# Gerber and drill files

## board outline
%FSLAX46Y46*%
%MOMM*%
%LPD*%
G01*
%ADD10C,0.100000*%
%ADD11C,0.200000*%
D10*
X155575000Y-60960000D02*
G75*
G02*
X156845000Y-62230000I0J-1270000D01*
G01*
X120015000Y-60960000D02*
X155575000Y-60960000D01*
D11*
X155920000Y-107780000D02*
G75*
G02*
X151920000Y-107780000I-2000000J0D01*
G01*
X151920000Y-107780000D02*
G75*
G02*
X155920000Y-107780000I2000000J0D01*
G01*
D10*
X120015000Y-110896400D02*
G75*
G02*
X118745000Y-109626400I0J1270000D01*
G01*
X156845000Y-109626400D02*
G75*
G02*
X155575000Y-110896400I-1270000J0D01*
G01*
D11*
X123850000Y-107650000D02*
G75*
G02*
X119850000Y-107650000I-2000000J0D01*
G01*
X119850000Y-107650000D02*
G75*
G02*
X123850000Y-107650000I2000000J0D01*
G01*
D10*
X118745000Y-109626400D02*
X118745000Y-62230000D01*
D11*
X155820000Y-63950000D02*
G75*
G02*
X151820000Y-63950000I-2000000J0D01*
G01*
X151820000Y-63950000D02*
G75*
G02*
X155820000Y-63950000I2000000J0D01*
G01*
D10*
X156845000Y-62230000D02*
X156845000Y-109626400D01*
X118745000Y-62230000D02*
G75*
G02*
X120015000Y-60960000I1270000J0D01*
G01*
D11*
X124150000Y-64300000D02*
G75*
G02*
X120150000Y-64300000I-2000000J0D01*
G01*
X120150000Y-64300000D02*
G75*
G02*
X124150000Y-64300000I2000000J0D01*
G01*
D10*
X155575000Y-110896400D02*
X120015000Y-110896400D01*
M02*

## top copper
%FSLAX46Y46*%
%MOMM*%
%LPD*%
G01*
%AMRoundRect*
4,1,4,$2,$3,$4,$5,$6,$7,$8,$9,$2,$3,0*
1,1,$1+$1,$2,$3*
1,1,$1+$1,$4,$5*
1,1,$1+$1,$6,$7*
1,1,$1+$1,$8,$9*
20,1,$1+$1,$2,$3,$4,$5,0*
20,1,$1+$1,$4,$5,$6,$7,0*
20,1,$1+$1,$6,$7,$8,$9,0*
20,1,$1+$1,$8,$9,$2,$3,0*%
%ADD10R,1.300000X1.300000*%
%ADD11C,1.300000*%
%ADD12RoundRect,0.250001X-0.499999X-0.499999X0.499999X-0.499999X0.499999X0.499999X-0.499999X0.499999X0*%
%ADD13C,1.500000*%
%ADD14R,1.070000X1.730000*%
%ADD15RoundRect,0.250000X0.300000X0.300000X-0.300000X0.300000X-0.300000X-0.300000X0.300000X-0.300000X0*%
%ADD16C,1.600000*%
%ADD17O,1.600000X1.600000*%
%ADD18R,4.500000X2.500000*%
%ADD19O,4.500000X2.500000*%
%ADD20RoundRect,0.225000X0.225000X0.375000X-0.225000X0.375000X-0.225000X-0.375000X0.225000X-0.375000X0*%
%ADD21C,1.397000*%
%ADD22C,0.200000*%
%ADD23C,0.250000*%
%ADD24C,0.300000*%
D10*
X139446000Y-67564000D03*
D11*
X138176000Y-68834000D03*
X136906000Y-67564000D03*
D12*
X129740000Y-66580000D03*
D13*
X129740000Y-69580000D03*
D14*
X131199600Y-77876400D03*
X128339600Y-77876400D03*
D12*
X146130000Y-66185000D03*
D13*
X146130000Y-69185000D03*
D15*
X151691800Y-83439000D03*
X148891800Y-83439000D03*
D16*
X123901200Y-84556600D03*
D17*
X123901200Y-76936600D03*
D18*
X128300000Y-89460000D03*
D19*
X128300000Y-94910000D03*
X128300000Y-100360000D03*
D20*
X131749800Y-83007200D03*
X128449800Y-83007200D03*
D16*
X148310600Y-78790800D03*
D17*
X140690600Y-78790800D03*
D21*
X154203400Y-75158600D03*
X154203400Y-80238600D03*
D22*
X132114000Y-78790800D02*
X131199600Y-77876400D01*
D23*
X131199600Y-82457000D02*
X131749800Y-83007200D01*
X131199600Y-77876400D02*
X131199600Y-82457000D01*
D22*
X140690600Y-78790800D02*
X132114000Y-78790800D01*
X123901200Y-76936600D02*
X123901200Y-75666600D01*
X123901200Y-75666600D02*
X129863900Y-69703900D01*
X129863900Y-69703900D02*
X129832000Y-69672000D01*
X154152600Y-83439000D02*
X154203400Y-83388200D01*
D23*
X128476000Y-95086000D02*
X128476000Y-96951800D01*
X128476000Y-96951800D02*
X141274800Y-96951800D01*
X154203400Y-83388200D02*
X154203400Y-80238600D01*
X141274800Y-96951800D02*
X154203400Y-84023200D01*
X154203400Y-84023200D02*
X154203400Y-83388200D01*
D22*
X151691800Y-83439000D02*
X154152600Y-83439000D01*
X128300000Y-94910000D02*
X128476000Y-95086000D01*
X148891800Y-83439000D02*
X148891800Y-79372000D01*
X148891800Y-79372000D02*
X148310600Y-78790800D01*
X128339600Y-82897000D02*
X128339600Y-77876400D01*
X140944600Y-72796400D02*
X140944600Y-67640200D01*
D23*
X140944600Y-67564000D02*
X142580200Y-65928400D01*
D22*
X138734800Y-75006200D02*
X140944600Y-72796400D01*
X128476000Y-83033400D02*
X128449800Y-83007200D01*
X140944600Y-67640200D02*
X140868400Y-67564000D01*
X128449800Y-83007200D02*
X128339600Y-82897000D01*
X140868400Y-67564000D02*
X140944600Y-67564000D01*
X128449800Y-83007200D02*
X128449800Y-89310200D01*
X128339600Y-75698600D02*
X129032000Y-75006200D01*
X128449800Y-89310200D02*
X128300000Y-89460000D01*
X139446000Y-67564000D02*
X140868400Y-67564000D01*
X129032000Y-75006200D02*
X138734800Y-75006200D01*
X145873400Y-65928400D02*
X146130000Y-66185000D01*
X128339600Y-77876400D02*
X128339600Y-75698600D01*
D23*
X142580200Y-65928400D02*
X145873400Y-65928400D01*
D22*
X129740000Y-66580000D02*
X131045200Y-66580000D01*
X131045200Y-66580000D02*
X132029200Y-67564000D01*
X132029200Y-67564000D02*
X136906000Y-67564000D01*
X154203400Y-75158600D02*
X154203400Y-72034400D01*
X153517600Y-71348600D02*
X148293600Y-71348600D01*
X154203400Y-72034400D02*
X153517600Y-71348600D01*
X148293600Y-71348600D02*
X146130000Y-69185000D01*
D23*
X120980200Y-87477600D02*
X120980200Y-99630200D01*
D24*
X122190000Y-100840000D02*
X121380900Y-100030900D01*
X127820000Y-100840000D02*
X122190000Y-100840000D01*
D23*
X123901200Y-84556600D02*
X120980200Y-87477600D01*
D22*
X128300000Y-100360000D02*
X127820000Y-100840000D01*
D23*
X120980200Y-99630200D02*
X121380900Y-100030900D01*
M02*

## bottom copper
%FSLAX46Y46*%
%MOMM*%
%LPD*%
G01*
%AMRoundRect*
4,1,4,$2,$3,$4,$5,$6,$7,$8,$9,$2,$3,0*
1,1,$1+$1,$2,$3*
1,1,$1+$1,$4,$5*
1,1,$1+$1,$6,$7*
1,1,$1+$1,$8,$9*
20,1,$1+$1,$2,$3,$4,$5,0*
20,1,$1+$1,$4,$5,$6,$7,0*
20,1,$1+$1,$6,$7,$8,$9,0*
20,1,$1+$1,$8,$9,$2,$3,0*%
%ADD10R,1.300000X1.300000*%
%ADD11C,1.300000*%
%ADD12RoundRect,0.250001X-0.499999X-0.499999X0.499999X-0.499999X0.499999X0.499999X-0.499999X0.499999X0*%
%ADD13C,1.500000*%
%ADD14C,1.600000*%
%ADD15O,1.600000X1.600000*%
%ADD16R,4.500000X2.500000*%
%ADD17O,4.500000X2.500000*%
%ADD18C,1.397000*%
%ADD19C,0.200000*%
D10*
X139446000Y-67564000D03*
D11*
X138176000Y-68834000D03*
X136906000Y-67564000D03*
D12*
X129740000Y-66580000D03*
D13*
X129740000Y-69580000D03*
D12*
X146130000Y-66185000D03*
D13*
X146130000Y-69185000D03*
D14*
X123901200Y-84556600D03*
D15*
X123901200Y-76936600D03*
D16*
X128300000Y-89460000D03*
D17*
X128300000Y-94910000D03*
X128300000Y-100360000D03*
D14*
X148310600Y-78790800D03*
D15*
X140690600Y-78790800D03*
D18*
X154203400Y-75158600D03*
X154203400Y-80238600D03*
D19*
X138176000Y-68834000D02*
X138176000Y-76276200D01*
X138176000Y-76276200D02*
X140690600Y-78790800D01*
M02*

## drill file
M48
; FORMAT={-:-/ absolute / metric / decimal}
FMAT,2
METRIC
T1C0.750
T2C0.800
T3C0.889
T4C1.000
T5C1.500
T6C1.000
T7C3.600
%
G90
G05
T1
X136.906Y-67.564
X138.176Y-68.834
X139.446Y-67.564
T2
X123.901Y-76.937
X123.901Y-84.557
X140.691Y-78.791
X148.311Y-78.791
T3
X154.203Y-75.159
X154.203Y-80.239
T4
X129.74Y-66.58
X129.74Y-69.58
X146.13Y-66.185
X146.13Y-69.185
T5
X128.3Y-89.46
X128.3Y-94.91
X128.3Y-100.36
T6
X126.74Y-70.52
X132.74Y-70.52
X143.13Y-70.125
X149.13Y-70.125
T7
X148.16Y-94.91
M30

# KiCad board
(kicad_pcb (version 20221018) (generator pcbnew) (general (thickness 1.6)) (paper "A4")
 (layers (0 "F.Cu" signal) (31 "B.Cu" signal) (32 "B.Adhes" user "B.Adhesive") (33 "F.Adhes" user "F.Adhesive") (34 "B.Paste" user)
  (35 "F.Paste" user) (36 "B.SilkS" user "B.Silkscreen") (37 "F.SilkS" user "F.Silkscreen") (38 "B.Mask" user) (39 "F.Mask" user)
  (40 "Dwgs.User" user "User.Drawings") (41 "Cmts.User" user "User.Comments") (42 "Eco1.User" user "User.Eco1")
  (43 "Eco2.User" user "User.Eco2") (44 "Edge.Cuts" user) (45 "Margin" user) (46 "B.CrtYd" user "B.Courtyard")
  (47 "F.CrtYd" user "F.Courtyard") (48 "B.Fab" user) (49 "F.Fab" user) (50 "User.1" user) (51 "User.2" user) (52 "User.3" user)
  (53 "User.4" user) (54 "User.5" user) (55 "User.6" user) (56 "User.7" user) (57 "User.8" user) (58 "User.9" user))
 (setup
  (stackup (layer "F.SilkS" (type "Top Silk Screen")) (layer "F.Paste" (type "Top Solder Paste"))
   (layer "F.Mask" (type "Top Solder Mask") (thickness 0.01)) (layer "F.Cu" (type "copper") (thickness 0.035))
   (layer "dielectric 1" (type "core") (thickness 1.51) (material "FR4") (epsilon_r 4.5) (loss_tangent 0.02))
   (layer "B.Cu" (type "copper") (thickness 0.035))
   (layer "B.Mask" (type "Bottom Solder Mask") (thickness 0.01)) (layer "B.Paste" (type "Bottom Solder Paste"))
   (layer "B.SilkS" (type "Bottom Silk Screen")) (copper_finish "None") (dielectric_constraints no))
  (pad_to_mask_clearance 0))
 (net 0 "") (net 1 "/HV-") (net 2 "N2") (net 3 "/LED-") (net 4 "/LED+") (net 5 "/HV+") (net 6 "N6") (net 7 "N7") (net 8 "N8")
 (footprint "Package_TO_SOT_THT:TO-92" (layer "F.Cu") (at 139.446 67.564 180)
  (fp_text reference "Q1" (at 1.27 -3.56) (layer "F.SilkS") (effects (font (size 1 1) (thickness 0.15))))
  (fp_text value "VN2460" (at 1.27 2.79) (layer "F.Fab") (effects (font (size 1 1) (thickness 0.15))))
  (pad "1" thru_hole rect (at 0 0 180) (size 1.3 1.3) (drill 0.75) (layers "*.Cu" "*.Mask") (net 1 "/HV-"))
  (pad "2" thru_hole circle (at 1.27 -1.27 180) (size 1.3 1.3) (drill 0.75) (layers "*.Cu" "*.Mask") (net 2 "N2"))
  (pad "3" thru_hole circle (at 2.54 0 180) (size 1.3 1.3) (drill 0.75) (layers "*.Cu" "*.Mask") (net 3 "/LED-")))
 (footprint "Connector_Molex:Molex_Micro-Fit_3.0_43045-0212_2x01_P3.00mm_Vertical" (layer "F.Cu") (at 129.74 66.58)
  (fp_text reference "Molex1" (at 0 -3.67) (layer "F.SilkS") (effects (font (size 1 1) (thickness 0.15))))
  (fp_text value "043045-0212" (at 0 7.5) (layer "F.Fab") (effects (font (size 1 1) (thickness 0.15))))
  (pad "" np_thru_hole circle (at -3 3.94) (size 1 1) (drill 1) (layers "*.Cu" "*.Mask"))
  (pad "" np_thru_hole circle (at 3 3.94) (size 1 1) (drill 1) (layers "*.Cu" "*.Mask"))
  (pad "1" thru_hole roundrect (at 0 0) (size 1.5 1.5) (drill 1) (layers "*.Cu" "*.Mask") (roundrect_rratio 0.166667) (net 3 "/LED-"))
  (pad "2" thru_hole circle (at 0 3) (size 1.5 1.5) (drill 1) (layers "*.Cu" "*.Mask") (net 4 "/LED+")))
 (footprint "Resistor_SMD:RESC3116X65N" (layer "F.Cu") (at 129.7696 77.8764 180)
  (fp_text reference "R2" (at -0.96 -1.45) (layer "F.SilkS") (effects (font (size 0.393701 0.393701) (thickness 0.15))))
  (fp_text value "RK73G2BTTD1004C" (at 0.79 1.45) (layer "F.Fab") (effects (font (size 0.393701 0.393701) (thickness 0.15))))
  (pad "1" smd rect (at -1.43 0 180) (size 1.07 1.73) (layers "F.Cu" "F.Paste" "F.Mask") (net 2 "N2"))
  (pad "2" smd rect (at 1.43 0 180) (size 1.07 1.73) (layers "F.Cu" "F.Paste" "F.Mask") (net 1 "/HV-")))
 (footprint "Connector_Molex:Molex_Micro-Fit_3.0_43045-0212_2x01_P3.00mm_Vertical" (layer "F.Cu") (at 146.13 66.185)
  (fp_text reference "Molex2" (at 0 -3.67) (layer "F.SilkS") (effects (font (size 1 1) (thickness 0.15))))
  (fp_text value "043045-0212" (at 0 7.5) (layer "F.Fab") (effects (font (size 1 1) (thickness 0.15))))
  (pad "" np_thru_hole circle (at -3 3.94) (size 1 1) (drill 1) (layers "*.Cu" "*.Mask"))
  (pad "" np_thru_hole circle (at 3 3.94) (size 1 1) (drill 1) (layers "*.Cu" "*.Mask"))
  (pad "1" thru_hole roundrect (at 0 0) (size 1.5 1.5) (drill 1) (layers "*.Cu" "*.Mask") (roundrect_rratio 0.166667) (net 1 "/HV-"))
  (pad "2" thru_hole circle (at 0 3) (size 1.5 1.5) (drill 1) (layers "*.Cu" "*.Mask") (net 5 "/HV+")))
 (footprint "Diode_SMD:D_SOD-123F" (layer "F.Cu") (at 150.2918 83.439 180)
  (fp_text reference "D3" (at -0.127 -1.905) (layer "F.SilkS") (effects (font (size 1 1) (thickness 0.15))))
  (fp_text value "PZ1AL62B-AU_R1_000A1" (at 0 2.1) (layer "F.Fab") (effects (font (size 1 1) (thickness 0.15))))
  (pad "1" smd roundrect (at -1.4 0 180) (size 1.1 1.1) (layers "F.Cu" "F.Paste" "F.Mask") (roundrect_rratio 0.2272727273) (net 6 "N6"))
  (pad "2" smd roundrect (at 1.4 0 180) (size 1.1 1.1) (layers "F.Cu" "F.Paste" "F.Mask") (roundrect_rratio 0.2272727273) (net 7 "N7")))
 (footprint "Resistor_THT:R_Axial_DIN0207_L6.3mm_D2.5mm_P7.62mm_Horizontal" (layer "F.Cu") (at 123.9012 84.5566 90)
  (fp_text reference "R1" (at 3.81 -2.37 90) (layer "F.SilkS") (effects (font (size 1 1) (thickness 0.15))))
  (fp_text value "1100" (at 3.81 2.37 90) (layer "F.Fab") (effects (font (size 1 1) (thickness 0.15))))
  (pad "1" thru_hole circle (at 0 0 90) (size 1.6 1.6) (drill 0.8) (layers "*.Cu" "*.Mask") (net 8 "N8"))
  (pad "2" thru_hole oval (at 7.62 0 90) (size 1.6 1.6) (drill 0.8) (layers "*.Cu" "*.Mask") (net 4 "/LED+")))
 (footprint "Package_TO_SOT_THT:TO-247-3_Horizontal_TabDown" (layer "F.Cu") (at 128.3 89.46 -90)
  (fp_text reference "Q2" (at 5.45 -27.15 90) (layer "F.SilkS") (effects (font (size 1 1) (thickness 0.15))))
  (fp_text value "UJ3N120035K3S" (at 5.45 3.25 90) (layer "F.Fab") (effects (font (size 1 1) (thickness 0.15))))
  (pad "" np_thru_hole oval (at 5.45 -19.86 270) (size 3.6 3.6) (drill 3.6) (layers "*.Cu" "*.Mask"))
  (pad "1" thru_hole rect (at 0 0 270) (size 2.5 4.5) (drill 1.5) (layers "*.Cu" "*.Mask") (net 1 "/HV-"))
  (pad "2" thru_hole oval (at 5.45 0 270) (size 2.5 4.5) (drill 1.5) (layers "*.Cu" "*.Mask") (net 6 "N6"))
  (pad "3" thru_hole oval (at 10.9 0 270) (size 2.5 4.5) (drill 1.5) (layers "*.Cu" "*.Mask") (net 8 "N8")))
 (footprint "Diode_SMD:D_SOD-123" (layer "F.Cu") (at 130.0998 83.0072 180)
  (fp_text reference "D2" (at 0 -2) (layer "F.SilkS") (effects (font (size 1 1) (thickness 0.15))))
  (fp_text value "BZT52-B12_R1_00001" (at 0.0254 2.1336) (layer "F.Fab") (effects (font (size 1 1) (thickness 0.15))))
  (pad "1" smd roundrect (at -1.65 0 180) (size 0.9 1.2) (layers "F.Cu" "F.Paste" "F.Mask") (roundrect_rratio 0.25) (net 2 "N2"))
  (pad "2" smd roundrect (at 1.65 0 180) (size 0.9 1.2) (layers "F.Cu" "F.Paste" "F.Mask") (roundrect_rratio 0.25) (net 1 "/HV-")))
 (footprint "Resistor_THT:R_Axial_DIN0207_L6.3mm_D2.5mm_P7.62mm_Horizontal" (layer "F.Cu") (at 148.3106 78.7908 180)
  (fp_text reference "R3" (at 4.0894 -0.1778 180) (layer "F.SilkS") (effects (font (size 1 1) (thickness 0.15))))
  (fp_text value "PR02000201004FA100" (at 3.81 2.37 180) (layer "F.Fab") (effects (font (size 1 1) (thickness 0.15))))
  (pad "1" thru_hole circle (at 0 0 180) (size 1.6 1.6) (drill 0.8) (layers "*.Cu" "*.Mask") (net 7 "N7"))
  (pad "2" thru_hole oval (at 7.62 0 180) (size 1.6 1.6) (drill 0.8) (layers "*.Cu" "*.Mask") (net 2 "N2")))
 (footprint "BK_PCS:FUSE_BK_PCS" (layer "F.Cu") (at 154.2034 77.6986 -90)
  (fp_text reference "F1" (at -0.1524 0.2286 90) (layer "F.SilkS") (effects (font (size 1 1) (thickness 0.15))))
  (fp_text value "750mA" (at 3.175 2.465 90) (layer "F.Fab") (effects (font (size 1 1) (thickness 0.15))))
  (pad "1" thru_hole circle (at -2.54 0 270) (size 1.397 1.397) (drill 0.889) (layers "*.Cu" "*.Mask") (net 5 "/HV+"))
  (pad "2" thru_hole circle (at 2.54 0 270) (size 1.397 1.397) (drill 0.889) (layers "*.Cu" "*.Mask") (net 6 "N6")))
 (gr_arc (start 155.575 60.96) (mid 156.473026 61.331974) (end 156.845 62.23) (stroke (width 0.1) (type default)) (layer "Edge.Cuts"))
 (gr_line (start 120.015 60.96) (end 155.575 60.96) (stroke (width 0.1) (type default)) (layer "Edge.Cuts"))
 (gr_circle (center 153.92 107.78) (end 155.92 107.78) (stroke (width 0.2) (type default)) (fill none) (layer "Edge.Cuts"))
 (gr_arc (start 120.015 110.8964) (mid 119.116974 110.524426) (end 118.745 109.6264) (stroke (width 0.1) (type default)) (layer "Edge.Cuts"))
 (gr_arc (start 156.845 109.6264) (mid 156.473026 110.524426) (end 155.575 110.8964) (stroke (width 0.1) (type default)) (layer "Edge.Cuts"))
 (gr_circle (center 121.85 107.65) (end 123.85 107.65) (stroke (width 0.2) (type default)) (fill none) (layer "Edge.Cuts"))
 (gr_line (start 118.745 109.6264) (end 118.745 62.23) (stroke (width 0.1) (type default)) (layer "Edge.Cuts"))
 (gr_circle (center 153.82 63.95) (end 155.82 63.95) (stroke (width 0.2) (type default)) (fill none) (layer "Edge.Cuts"))
 (gr_line (start 156.845 62.23) (end 156.845 109.6264) (stroke (width 0.1) (type default)) (layer "Edge.Cuts"))
 (gr_arc (start 118.745 62.23) (mid 119.116974 61.331974) (end 120.015 60.96) (stroke (width 0.1) (type default)) (layer "Edge.Cuts"))
 (gr_circle (center 122.15 64.3) (end 124.15 64.3) (stroke (width 0.2) (type default)) (fill none) (layer "Edge.Cuts"))
 (gr_line (start 155.575 110.8964) (end 120.015 110.8964) (stroke (width 0.1) (type default)) (layer "Edge.Cuts"))
 (segment (start 132.114 78.7908) (end 131.1996 77.8764) (width 0.2) (layer "F.Cu") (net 2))
 (segment (start 131.1996 82.457) (end 131.7498 83.0072) (width 0.25) (layer "F.Cu") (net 2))
 (segment (start 131.1996 77.8764) (end 131.1996 82.457) (width 0.25) (layer "F.Cu") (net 2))
 (segment (start 140.6906 78.7908) (end 132.114 78.7908) (width 0.2) (layer "F.Cu") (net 2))
 (segment (start 138.176 68.834) (end 138.176 76.2762) (width 0.2) (layer "B.Cu") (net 2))
 (segment (start 138.176 76.2762) (end 140.6906 78.7908) (width 0.2) (layer "B.Cu") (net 2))
 (segment (start 123.9012 76.9366) (end 123.9012 75.6666) (width 0.2) (layer "F.Cu") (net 4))
 (segment (start 123.9012 75.6666) (end 129.8639 69.7039) (width 0.2) (layer "F.Cu") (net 4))
 (segment (start 129.8639 69.7039) (end 129.832 69.672) (width 0.2) (layer "F.Cu") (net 4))
 (segment (start 154.1526 83.439) (end 154.2034 83.3882) (width 0.2) (layer "F.Cu") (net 6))
 (segment (start 128.476 95.086) (end 128.476 96.9518) (width 0.25) (layer "F.Cu") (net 6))
 (segment (start 128.476 96.9518) (end 141.2748 96.9518) (width 0.25) (layer "F.Cu") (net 6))
 (segment (start 154.2034 83.3882) (end 154.2034 80.2386) (width 0.25) (layer "F.Cu") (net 6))
 (segment (start 141.2748 96.9518) (end 154.2034 84.0232) (width 0.25) (layer "F.Cu") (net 6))
 (segment (start 154.2034 84.0232) (end 154.2034 83.3882) (width 0.25) (layer "F.Cu") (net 6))
 (segment (start 151.6918 83.439) (end 154.1526 83.439) (width 0.2) (layer "F.Cu") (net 6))
 (segment (start 128.3 94.91) (end 128.476 95.086) (width 0.2) (layer "F.Cu") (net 6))
 (segment (start 148.8918 83.439) (end 148.8918 79.372) (width 0.2) (layer "F.Cu") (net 7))
 (segment (start 148.8918 79.372) (end 148.3106 78.7908) (width 0.2) (layer "F.Cu") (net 7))
 (segment (start 128.3396 82.897) (end 128.3396 77.8764) (width 0.2) (layer "F.Cu") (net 1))
 (segment (start 140.9446 72.7964) (end 140.9446 67.6402) (width 0.2) (layer "F.Cu") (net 1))
 (segment (start 140.9446 67.564) (end 142.5802 65.9284) (width 0.25) (layer "F.Cu") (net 1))
 (segment (start 138.7348 75.0062) (end 140.9446 72.7964) (width 0.2) (layer "F.Cu") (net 1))
 (segment (start 128.476 83.0334) (end 128.4498 83.0072) (width 0.2) (layer "F.Cu") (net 1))
 (segment (start 140.9446 67.6402) (end 140.8684 67.564) (width 0.2) (layer "F.Cu") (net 1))
 (segment (start 128.4498 83.0072) (end 128.3396 82.897) (width 0.2) (layer "F.Cu") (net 1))
 (segment (start 140.8684 67.564) (end 140.9446 67.564) (width 0.2) (layer "F.Cu") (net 1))
 (segment (start 128.4498 83.0072) (end 128.4498 89.3102) (width 0.2) (layer "F.Cu") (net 1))
 (segment (start 128.3396 75.6986) (end 129.032 75.0062) (width 0.2) (layer "F.Cu") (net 1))
 (segment (start 128.4498 89.3102) (end 128.3 89.46) (width 0.2) (layer "F.Cu") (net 1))
 (segment (start 139.446 67.564) (end 140.8684 67.564) (width 0.2) (layer "F.Cu") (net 1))
 (segment (start 129.032 75.0062) (end 138.7348 75.0062) (width 0.2) (layer "F.Cu") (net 1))
 (segment (start 145.8734 65.9284) (end 146.13 66.185) (width 0.2) (layer "F.Cu") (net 1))
 (segment (start 128.3396 77.8764) (end 128.3396 75.6986) (width 0.2) (layer "F.Cu") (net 1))
 (segment (start 142.5802 65.9284) (end 145.8734 65.9284) (width 0.25) (layer "F.Cu") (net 1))
 (segment (start 129.74 66.58) (end 131.0452 66.58) (width 0.2) (layer "F.Cu") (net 3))
 (segment (start 131.0452 66.58) (end 132.0292 67.564) (width 0.2) (layer "F.Cu") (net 3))
 (segment (start 132.0292 67.564) (end 136.906 67.564) (width 0.2) (layer "F.Cu") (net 3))
 (segment (start 154.2034 75.1586) (end 154.2034 72.0344) (width 0.2) (layer "F.Cu") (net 5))
 (segment (start 153.5176 71.3486) (end 148.2936 71.3486) (width 0.2) (layer "F.Cu") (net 5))
 (segment (start 154.2034 72.0344) (end 153.5176 71.3486) (width 0.2) (layer "F.Cu") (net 5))
 (segment (start 148.2936 71.3486) (end 146.13 69.185) (width 0.2) (layer "F.Cu") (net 5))
 (segment (start 120.9802 87.4776) (end 120.9802 99.6302) (width 0.25) (layer "F.Cu") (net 8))
 (segment (start 122.19 100.84) (end 121.3809 100.0309) (width 0.3) (layer "F.Cu") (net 8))
 (segment (start 127.82 100.84) (end 122.19 100.84) (width 0.3) (layer "F.Cu") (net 8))
 (segment (start 123.9012 84.5566) (end 120.9802 87.4776) (width 0.25) (layer "F.Cu") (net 8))
 (segment (start 128.3 100.36) (end 127.82 100.84) (width 0.2) (layer "F.Cu") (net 8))
 (segment (start 120.9802 99.6302) (end 121.3809 100.0309) (width 0.25) (layer "F.Cu") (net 8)))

